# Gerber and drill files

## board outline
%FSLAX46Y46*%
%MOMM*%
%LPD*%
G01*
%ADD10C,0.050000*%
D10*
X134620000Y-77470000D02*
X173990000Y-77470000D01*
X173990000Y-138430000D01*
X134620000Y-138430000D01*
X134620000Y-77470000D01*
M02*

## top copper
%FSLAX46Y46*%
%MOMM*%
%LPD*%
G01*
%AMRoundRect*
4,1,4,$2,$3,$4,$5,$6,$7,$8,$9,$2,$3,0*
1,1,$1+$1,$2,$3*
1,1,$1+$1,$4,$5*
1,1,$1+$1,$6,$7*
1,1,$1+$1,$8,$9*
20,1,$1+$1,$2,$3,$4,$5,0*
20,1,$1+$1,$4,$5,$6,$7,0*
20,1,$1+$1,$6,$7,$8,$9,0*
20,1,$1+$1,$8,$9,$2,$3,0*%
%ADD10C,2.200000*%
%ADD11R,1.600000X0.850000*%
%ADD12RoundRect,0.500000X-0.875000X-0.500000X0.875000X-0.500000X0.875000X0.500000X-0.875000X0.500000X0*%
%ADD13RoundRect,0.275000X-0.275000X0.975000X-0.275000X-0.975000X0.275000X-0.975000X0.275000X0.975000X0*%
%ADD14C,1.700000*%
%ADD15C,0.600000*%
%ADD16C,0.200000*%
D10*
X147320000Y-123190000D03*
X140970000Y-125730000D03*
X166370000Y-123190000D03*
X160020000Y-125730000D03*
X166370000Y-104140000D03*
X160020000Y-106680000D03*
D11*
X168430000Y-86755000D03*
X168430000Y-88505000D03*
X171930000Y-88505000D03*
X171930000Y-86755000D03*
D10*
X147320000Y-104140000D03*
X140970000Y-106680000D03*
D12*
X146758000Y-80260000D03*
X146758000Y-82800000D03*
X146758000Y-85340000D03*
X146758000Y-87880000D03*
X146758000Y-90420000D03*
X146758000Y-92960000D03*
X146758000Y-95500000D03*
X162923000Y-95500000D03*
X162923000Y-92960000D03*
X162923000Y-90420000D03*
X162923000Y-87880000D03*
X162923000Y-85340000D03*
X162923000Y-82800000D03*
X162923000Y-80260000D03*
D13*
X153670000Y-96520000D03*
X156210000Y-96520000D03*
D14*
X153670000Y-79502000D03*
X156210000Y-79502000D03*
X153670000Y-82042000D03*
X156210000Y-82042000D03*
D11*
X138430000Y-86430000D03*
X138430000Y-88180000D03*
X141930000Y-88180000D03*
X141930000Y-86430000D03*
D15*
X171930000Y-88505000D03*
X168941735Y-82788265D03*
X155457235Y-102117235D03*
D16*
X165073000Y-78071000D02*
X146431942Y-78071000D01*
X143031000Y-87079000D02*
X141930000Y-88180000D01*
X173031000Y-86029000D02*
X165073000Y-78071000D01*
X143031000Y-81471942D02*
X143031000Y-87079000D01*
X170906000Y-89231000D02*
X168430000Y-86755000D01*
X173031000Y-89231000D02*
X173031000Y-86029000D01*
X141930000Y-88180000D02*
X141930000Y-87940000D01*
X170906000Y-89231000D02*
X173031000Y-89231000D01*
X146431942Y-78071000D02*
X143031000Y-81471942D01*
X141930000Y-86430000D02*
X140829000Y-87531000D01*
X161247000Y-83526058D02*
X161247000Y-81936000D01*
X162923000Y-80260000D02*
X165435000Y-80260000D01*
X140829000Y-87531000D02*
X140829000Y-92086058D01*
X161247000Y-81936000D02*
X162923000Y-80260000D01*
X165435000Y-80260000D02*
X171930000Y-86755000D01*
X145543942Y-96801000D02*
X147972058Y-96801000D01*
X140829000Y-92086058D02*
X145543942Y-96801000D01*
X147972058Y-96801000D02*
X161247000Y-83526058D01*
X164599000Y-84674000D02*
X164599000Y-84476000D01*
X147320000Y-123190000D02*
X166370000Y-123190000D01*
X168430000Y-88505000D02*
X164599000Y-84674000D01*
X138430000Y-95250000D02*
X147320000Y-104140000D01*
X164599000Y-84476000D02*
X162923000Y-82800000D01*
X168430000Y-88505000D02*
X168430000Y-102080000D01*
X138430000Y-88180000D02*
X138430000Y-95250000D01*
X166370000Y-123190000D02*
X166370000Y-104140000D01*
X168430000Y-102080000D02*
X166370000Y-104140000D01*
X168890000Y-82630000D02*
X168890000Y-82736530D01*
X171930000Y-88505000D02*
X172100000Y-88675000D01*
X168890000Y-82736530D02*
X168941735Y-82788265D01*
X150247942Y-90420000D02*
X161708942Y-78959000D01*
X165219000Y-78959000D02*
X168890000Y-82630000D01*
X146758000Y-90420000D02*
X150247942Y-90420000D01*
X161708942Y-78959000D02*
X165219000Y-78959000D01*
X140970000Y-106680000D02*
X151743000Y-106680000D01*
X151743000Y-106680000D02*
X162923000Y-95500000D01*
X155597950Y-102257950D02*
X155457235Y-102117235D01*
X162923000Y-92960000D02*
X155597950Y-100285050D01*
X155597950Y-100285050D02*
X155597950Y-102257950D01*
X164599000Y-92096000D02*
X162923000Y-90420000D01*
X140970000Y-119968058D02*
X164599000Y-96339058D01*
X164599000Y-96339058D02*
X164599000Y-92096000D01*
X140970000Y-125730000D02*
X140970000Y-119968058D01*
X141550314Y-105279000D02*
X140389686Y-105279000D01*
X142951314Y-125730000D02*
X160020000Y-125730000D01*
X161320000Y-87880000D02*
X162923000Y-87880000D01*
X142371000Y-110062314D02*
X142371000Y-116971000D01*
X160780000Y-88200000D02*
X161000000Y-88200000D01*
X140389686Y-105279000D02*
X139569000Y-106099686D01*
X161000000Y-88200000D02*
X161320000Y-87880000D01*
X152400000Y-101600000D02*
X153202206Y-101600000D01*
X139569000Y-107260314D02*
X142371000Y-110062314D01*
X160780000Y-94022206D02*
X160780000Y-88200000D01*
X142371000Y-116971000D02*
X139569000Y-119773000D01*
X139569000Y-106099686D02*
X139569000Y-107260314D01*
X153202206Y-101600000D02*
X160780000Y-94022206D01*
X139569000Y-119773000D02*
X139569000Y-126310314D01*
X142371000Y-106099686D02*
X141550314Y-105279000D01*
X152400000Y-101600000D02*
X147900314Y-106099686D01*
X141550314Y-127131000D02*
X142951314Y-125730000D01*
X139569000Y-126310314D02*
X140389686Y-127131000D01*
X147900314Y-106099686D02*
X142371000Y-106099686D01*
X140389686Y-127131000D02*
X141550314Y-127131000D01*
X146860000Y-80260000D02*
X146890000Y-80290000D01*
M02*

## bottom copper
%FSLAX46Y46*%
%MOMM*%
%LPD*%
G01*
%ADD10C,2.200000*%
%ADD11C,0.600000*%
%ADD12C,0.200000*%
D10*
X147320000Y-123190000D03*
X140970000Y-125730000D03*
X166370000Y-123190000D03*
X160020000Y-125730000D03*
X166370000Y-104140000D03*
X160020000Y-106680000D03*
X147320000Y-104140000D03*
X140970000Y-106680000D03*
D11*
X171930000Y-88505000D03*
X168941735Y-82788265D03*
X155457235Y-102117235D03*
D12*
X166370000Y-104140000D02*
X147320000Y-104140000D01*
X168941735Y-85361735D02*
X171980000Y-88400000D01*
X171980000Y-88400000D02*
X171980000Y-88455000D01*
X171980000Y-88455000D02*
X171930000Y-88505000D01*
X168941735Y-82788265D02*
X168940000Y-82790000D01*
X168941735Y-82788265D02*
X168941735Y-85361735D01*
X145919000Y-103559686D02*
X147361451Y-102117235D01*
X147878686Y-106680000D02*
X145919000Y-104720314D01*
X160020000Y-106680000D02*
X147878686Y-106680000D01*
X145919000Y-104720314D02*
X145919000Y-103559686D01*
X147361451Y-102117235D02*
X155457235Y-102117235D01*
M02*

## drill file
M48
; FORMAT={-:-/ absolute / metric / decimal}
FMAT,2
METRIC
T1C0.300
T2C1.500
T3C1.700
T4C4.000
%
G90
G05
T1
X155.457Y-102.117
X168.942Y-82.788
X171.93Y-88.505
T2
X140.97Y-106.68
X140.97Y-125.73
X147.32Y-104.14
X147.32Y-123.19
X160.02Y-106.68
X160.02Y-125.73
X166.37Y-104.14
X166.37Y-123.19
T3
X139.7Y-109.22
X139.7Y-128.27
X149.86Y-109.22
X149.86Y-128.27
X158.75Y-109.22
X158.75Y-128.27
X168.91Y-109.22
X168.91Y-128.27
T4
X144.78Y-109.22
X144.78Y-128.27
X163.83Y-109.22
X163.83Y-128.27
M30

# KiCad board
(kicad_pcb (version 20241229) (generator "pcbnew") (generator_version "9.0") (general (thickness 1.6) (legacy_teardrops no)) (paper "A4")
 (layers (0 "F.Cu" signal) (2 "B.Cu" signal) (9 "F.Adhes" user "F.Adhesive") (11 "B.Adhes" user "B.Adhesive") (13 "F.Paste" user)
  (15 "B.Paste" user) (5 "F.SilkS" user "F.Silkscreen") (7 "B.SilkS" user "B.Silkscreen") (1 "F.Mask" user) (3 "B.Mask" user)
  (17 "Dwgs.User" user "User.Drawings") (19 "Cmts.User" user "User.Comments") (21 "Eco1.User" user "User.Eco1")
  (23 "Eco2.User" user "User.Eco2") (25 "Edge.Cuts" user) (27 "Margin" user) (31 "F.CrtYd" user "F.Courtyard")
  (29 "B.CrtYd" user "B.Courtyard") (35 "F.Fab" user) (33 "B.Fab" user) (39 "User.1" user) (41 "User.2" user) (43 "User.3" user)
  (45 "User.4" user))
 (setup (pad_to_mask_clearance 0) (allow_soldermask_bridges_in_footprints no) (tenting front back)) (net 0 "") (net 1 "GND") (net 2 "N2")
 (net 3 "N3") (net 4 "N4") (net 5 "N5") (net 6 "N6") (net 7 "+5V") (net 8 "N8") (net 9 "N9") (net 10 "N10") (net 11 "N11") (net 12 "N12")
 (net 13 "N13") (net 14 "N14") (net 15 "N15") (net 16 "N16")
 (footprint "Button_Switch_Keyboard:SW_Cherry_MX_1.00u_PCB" (layer "F.Cu") (at 147.32 123.19)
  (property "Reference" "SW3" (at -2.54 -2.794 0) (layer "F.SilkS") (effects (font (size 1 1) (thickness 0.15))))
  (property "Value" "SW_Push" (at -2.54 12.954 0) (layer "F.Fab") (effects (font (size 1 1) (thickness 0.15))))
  (pad "" np_thru_hole circle (at -7.62 5.08) (size 1.7 1.7) (drill 1.7) (layers "*.Cu" "*.Mask"))
  (pad "" np_thru_hole circle (at -2.54 5.08) (size 4 4) (drill 4) (layers "*.Cu" "*.Mask"))
  (pad "" np_thru_hole circle (at 2.54 5.08) (size 1.7 1.7) (drill 1.7) (layers "*.Cu" "*.Mask"))
  (pad "1" thru_hole circle (at 0 0) (size 2.2 2.2) (drill 1.5) (layers "*.Cu" "*.Mask") (remove_unused_layers no) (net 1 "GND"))
  (pad "2" thru_hole circle (at -6.35 2.54) (size 2.2 2.2) (drill 1.5) (layers "*.Cu" "*.Mask") (remove_unused_layers no) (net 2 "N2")))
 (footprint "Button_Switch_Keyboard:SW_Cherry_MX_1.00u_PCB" (layer "F.Cu") (at 166.37 123.19)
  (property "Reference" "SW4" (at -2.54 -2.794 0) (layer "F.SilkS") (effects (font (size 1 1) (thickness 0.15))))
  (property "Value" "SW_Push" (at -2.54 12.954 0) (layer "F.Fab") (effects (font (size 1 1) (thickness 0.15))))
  (pad "" np_thru_hole circle (at -7.62 5.08) (size 1.7 1.7) (drill 1.7) (layers "*.Cu" "*.Mask"))
  (pad "" np_thru_hole circle (at -2.54 5.08) (size 4 4) (drill 4) (layers "*.Cu" "*.Mask"))
  (pad "" np_thru_hole circle (at 2.54 5.08) (size 1.7 1.7) (drill 1.7) (layers "*.Cu" "*.Mask"))
  (pad "1" thru_hole circle (at 0 0) (size 2.2 2.2) (drill 1.5) (layers "*.Cu" "*.Mask") (remove_unused_layers no) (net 1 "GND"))
  (pad "2" thru_hole circle (at -6.35 2.54) (size 2.2 2.2) (drill 1.5) (layers "*.Cu" "*.Mask") (remove_unused_layers no) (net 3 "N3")))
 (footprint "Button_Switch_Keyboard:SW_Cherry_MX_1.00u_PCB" (layer "F.Cu") (at 166.37 104.14)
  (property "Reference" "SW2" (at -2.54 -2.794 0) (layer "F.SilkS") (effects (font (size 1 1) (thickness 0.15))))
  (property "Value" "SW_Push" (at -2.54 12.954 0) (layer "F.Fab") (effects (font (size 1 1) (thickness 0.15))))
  (pad "" np_thru_hole circle (at -7.62 5.08) (size 1.7 1.7) (drill 1.7) (layers "*.Cu" "*.Mask"))
  (pad "" np_thru_hole circle (at -2.54 5.08) (size 4 4) (drill 4) (layers "*.Cu" "*.Mask"))
  (pad "" np_thru_hole circle (at 2.54 5.08) (size 1.7 1.7) (drill 1.7) (layers "*.Cu" "*.Mask"))
  (pad "1" thru_hole circle (at 0 0) (size 2.2 2.2) (drill 1.5) (layers "*.Cu" "*.Mask") (remove_unused_layers no) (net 1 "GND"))
  (pad "2" thru_hole circle (at -6.35 2.54) (size 2.2 2.2) (drill 1.5) (layers "*.Cu" "*.Mask") (remove_unused_layers no) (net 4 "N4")))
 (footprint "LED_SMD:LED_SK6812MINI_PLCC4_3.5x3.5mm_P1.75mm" (layer "F.Cu") (at 170.18 87.63)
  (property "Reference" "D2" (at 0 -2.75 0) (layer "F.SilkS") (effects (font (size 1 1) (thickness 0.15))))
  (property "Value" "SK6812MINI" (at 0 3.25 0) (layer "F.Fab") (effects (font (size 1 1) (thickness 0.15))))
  (pad "1" smd rect (at -1.75 -0.875) (size 1.6 0.85) (layers "F.Cu" "F.Mask" "F.Paste") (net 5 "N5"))
  (pad "2" smd rect (at -1.75 0.875) (size 1.6 0.85) (layers "F.Cu" "F.Mask" "F.Paste") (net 1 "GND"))
  (pad "3" smd rect (at 1.75 0.875) (size 1.6 0.85) (layers "F.Cu" "F.Mask" "F.Paste") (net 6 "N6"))
  (pad "4" smd rect (at 1.75 -0.875) (size 1.6 0.85) (layers "F.Cu" "F.Mask" "F.Paste") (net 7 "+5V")))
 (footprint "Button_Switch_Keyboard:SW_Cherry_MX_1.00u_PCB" (layer "F.Cu") (at 147.32 104.14)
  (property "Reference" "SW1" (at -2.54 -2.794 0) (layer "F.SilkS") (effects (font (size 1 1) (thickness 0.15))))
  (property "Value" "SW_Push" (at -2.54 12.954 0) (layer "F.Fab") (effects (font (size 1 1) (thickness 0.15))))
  (pad "" np_thru_hole circle (at -7.62 5.08) (size 1.7 1.7) (drill 1.7) (layers "*.Cu" "*.Mask"))
  (pad "" np_thru_hole circle (at -2.54 5.08) (size 4 4) (drill 4) (layers "*.Cu" "*.Mask"))
  (pad "" np_thru_hole circle (at 2.54 5.08) (size 1.7 1.7) (drill 1.7) (layers "*.Cu" "*.Mask"))
  (pad "1" thru_hole circle (at 0 0) (size 2.2 2.2) (drill 1.5) (layers "*.Cu" "*.Mask") (remove_unused_layers no) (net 1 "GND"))
  (pad "2" thru_hole circle (at -6.35 2.54) (size 2.2 2.2) (drill 1.5) (layers "*.Cu" "*.Mask") (remove_unused_layers no) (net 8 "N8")))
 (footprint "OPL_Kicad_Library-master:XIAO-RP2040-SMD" (layer "F.Cu") (at 154.758 87.88)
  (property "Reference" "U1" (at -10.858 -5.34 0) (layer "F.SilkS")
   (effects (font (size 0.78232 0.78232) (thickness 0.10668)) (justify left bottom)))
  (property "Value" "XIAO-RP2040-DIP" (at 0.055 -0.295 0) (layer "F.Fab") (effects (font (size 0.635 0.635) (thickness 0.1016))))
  (pad "1" smd roundrect (at -8 -7.62) (size 2.75 2) (layers "F.Cu" "F.Mask" "F.Paste") (roundrect_rratio 0.25) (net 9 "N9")
   (solder_mask_margin 0.0508) (thermal_bridge_angle 45))
  (pad "2" smd roundrect (at -8 -5.08) (size 2.75 2) (layers "F.Cu" "F.Mask" "F.Paste") (roundrect_rratio 0.25) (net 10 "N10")
   (solder_mask_margin 0.0508) (thermal_bridge_angle 45))
  (pad "3" smd roundrect (at -8 -2.54) (size 2.75 2) (layers "F.Cu" "F.Mask" "F.Paste") (roundrect_rratio 0.25) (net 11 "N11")
   (solder_mask_margin 0.0508) (thermal_bridge_angle 45))
  (pad "4" smd roundrect (at -8 0) (size 2.75 2) (layers "F.Cu" "F.Mask" "F.Paste") (roundrect_rratio 0.25) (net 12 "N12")
   (solder_mask_margin 0.0508) (thermal_bridge_angle 45))
  (pad "5" smd roundrect (at -8 2.54) (size 2.75 2) (layers "F.Cu" "F.Mask" "F.Paste") (roundrect_rratio 0.25) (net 6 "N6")
   (solder_mask_margin 0.0508) (thermal_bridge_angle 45))
  (pad "6" smd roundrect (at -8 5.08) (size 2.75 2) (layers "F.Cu" "F.Mask" "F.Paste") (roundrect_rratio 0.25) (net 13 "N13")
   (solder_mask_margin 0.0508) (thermal_bridge_angle 45))
  (pad "7" smd roundrect (at -8 7.62) (size 2.75 2) (layers "F.Cu" "F.Mask" "F.Paste") (roundrect_rratio 0.25) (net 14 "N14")
   (solder_mask_margin 0.0508) (thermal_bridge_angle 45))
  (pad "8" smd roundrect (at 8.165 7.62) (size 2.75 2) (layers "F.Cu" "F.Mask" "F.Paste") (roundrect_rratio 0.25) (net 8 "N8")
   (solder_mask_margin 0.0508) (thermal_bridge_angle 45))
  (pad "9" smd roundrect (at 8.165 5.08) (size 2.75 2) (layers "F.Cu" "F.Mask" "F.Paste") (roundrect_rratio 0.25) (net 4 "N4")
   (solder_mask_margin 0.0508) (thermal_bridge_angle 45))
  (pad "10" smd roundrect (at 8.165 2.54) (size 2.75 2) (layers "F.Cu" "F.Mask" "F.Paste") (roundrect_rratio 0.25) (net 2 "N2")
   (solder_mask_margin 0.0508) (thermal_bridge_angle 45))
  (pad "11" smd roundrect (at 8.165 0) (size 2.75 2) (layers "F.Cu" "F.Mask" "F.Paste") (roundrect_rratio 0.25) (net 3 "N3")
   (solder_mask_margin 0.0508) (thermal_bridge_angle 45))
  (pad "12" smd roundrect (at 8.165 -2.54) (size 2.75 2) (layers "F.Cu" "F.Mask" "F.Paste") (roundrect_rratio 0.25) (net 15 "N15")
   (solder_mask_margin 0.0508) (thermal_bridge_angle 45))
  (pad "13" smd roundrect (at 8.165 -5.08) (size 2.75 2) (layers "F.Cu" "F.Mask" "F.Paste") (roundrect_rratio 0.25) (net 1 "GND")
   (solder_mask_margin 0.0508) (thermal_bridge_angle 45))
  (pad "14" smd roundrect (at 8.165 -7.62) (size 2.75 2) (layers "F.Cu" "F.Mask" "F.Paste") (roundrect_rratio 0.25) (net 7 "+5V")
   (solder_mask_margin 0.0508) (thermal_bridge_angle 45))
  (pad "15" smd roundrect (at -1.088 8.64 270) (size 2.5 1.1) (layers "F.Cu" "F.Mask" "F.Paste") (roundrect_rratio 0.25)
   (thermal_bridge_angle 45))
  (pad "16" smd roundrect (at 1.452 8.64 270) (size 2.5 1.1) (layers "F.Cu" "F.Mask" "F.Paste") (roundrect_rratio 0.25)
   (thermal_bridge_angle 45))
  (pad "17" smd circle (at -1.088 -8.378) (size 1.7 1.7) (layers "F.Cu" "F.Mask" "F.Paste"))
  (pad "18" smd circle (at 1.452 -8.378) (size 1.7 1.7) (layers "F.Cu" "F.Mask" "F.Paste"))
  (pad "19" smd circle (at -1.088 -5.838) (size 1.7 1.7) (layers "F.Cu" "F.Mask" "F.Paste"))
  (pad "20" smd circle (at 1.452 -5.838) (size 1.7 1.7) (layers "F.Cu" "F.Mask" "F.Paste")))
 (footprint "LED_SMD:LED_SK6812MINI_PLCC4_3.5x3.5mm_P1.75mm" (layer "F.Cu") (at 140.18 87.305)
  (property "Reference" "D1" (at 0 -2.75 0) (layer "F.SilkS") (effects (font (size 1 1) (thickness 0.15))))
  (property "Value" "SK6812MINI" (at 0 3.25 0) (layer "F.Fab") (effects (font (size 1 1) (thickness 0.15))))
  (pad "1" smd rect (at -1.75 -0.875) (size 1.6 0.85) (layers "F.Cu" "F.Mask" "F.Paste") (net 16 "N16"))
  (pad "2" smd rect (at -1.75 0.875) (size 1.6 0.85) (layers "F.Cu" "F.Mask" "F.Paste") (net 1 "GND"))
  (pad "3" smd rect (at 1.75 0.875) (size 1.6 0.85) (layers "F.Cu" "F.Mask" "F.Paste") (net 5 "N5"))
  (pad "4" smd rect (at 1.75 -0.875) (size 1.6 0.85) (layers "F.Cu" "F.Mask" "F.Paste") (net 7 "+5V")))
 (gr_rect (start 134.62 77.47) (end 173.99 138.43) (stroke (width 0.05) (type default)) (fill no) (layer "Edge.Cuts"))
 (segment (start 165.073 78.071) (end 146.431942 78.071) (width 0.2) (layer "F.Cu") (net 5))
 (segment (start 143.031 87.079) (end 141.93 88.18) (width 0.2) (layer "F.Cu") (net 5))
 (segment (start 173.031 86.029) (end 165.073 78.071) (width 0.2) (layer "F.Cu") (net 5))
 (segment (start 143.031 81.471942) (end 143.031 87.079) (width 0.2) (layer "F.Cu") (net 5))
 (segment (start 170.906 89.231) (end 168.43 86.755) (width 0.2) (layer "F.Cu") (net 5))
 (segment (start 173.031 89.231) (end 173.031 86.029) (width 0.2) (layer "F.Cu") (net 5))
 (segment (start 141.93 88.18) (end 141.93 87.94) (width 0.2) (layer "F.Cu") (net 5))
 (segment (start 170.906 89.231) (end 173.031 89.231) (width 0.2) (layer "F.Cu") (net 5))
 (segment (start 146.431942 78.071) (end 143.031 81.471942) (width 0.2) (layer "F.Cu") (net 5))
 (segment (start 141.93 86.43) (end 140.829 87.531) (width 0.2) (layer "F.Cu") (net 7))
 (segment (start 161.247 83.526058) (end 161.247 81.936) (width 0.2) (layer "F.Cu") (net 7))
 (segment (start 162.923 80.26) (end 165.435 80.26) (width 0.2) (layer "F.Cu") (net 7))
 (segment (start 140.829 87.531) (end 140.829 92.086058) (width 0.2) (layer "F.Cu") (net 7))
 (segment (start 161.247 81.936) (end 162.923 80.26) (width 0.2) (layer "F.Cu") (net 7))
 (segment (start 165.435 80.26) (end 171.93 86.755) (width 0.2) (layer "F.Cu") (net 7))
 (segment (start 145.543942 96.801) (end 147.972058 96.801) (width 0.2) (layer "F.Cu") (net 7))
 (segment (start 140.829 92.086058) (end 145.543942 96.801) (width 0.2) (layer "F.Cu") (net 7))
 (segment (start 147.972058 96.801) (end 161.247 83.526058) (width 0.2) (layer "F.Cu") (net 7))
 (segment (start 164.599 84.674) (end 164.599 84.476) (width 0.2) (layer "F.Cu") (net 1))
 (segment (start 147.32 123.19) (end 166.37 123.19) (width 0.2) (layer "F.Cu") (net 1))
 (segment (start 168.43 88.505) (end 164.599 84.674) (width 0.2) (layer "F.Cu") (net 1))
 (segment (start 138.43 95.25) (end 147.32 104.14) (width 0.2) (layer "F.Cu") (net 1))
 (segment (start 164.599 84.476) (end 162.923 82.8) (width 0.2) (layer "F.Cu") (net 1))
 (segment (start 168.43 88.505) (end 168.43 102.08) (width 0.2) (layer "F.Cu") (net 1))
 (segment (start 138.43 88.18) (end 138.43 95.25) (width 0.2) (layer "F.Cu") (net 1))
 (segment (start 166.37 123.19) (end 166.37 104.14) (width 0.2) (layer "F.Cu") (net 1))
 (segment (start 168.43 102.08) (end 166.37 104.14) (width 0.2) (layer "F.Cu") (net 1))
 (segment (start 166.37 104.14) (end 147.32 104.14) (width 0.2) (layer "B.Cu") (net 1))
 (segment (start 168.89 82.63) (end 168.89 82.73653) (width 0.2) (layer "F.Cu") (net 6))
 (segment (start 171.93 88.505) (end 172.1 88.675) (width 0.2) (layer "F.Cu") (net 6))
 (segment (start 168.89 82.73653) (end 168.941735 82.788265) (width 0.2) (layer "F.Cu") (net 6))
 (segment (start 150.247942 90.42) (end 161.708942 78.959) (width 0.2) (layer "F.Cu") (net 6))
 (segment (start 165.219 78.959) (end 168.89 82.63) (width 0.2) (layer "F.Cu") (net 6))
 (segment (start 146.758 90.42) (end 150.247942 90.42) (width 0.2) (layer "F.Cu") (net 6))
 (segment (start 161.708942 78.959) (end 165.219 78.959) (width 0.2) (layer "F.Cu") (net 6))
 (via (at 171.93 88.505) (size 0.6) (drill 0.3) (layers "F.Cu" "B.Cu") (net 6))
 (via (at 168.941735 82.788265) (size 0.6) (drill 0.3) (layers "F.Cu" "B.Cu") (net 6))
 (segment (start 168.941735 85.361735) (end 171.98 88.4) (width 0.2) (layer "B.Cu") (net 6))
 (segment (start 171.98 88.4) (end 171.98 88.455) (width 0.2) (layer "B.Cu") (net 6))
 (segment (start 171.98 88.455) (end 171.93 88.505) (width 0.2) (layer "B.Cu") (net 6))
 (segment (start 168.941735 82.788265) (end 168.94 82.79) (width 0.2) (layer "B.Cu") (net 6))
 (segment (start 168.941735 82.788265) (end 168.941735 85.361735) (width 0.2) (layer "B.Cu") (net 6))
 (segment (start 140.97 106.68) (end 151.743 106.68) (width 0.2) (layer "F.Cu") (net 8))
 (segment (start 151.743 106.68) (end 162.923 95.5) (width 0.2) (layer "F.Cu") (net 8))
 (segment (start 155.59795 102.25795) (end 155.457235 102.117235) (width 0.2) (layer "F.Cu") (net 4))
 (segment (start 162.923 92.96) (end 155.59795 100.28505) (width 0.2) (layer "F.Cu") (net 4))
 (segment (start 155.59795 100.28505) (end 155.59795 102.25795) (width 0.2) (layer "F.Cu") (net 4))
 (via (at 155.457235 102.117235) (size 0.6) (drill 0.3) (layers "F.Cu" "B.Cu") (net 4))
 (segment (start 145.919 103.559686) (end 147.361451 102.117235) (width 0.2) (layer "B.Cu") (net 4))
 (segment (start 147.878686 106.68) (end 145.919 104.720314) (width 0.2) (layer "B.Cu") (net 4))
 (segment (start 160.02 106.68) (end 147.878686 106.68) (width 0.2) (layer "B.Cu") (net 4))
 (segment (start 145.919 104.720314) (end 145.919 103.559686) (width 0.2) (layer "B.Cu") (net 4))
 (segment (start 147.361451 102.117235) (end 155.457235 102.117235) (width 0.2) (layer "B.Cu") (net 4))
 (segment (start 164.599 92.096) (end 162.923 90.42) (width 0.2) (layer "F.Cu") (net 2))
 (segment (start 140.97 119.968058) (end 164.599 96.339058) (width 0.2) (layer "F.Cu") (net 2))
 (segment (start 164.599 96.339058) (end 164.599 92.096) (width 0.2) (layer "F.Cu") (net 2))
 (segment (start 140.97 125.73) (end 140.97 119.968058) (width 0.2) (layer "F.Cu") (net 2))
 (segment (start 141.550314 105.279) (end 140.389686 105.279) (width 0.2) (layer "F.Cu") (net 3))
 (segment (start 142.951314 125.73) (end 160.02 125.73) (width 0.2) (layer "F.Cu") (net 3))
 (segment (start 161.32 87.88) (end 162.923 87.88) (width 0.2) (layer "F.Cu") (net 3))
 (segment (start 142.371 110.062314) (end 142.371 116.971) (width 0.2) (layer "F.Cu") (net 3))
 (segment (start 160.78 88.2) (end 161 88.2) (width 0.2) (layer "F.Cu") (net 3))
 (segment (start 140.389686 105.279) (end 139.569 106.099686) (width 0.2) (layer "F.Cu") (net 3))
 (segment (start 161 88.2) (end 161.32 87.88) (width 0.2) (layer "F.Cu") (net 3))
 (segment (start 152.4 101.6) (end 153.202206 101.6) (width 0.2) (layer "F.Cu") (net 3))
 (segment (start 139.569 107.260314) (end 142.371 110.062314) (width 0.2) (layer "F.Cu") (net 3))
 (segment (start 160.78 94.022206) (end 160.78 88.2) (width 0.2) (layer "F.Cu") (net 3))
 (segment (start 142.371 116.971) (end 139.569 119.773) (width 0.2) (layer "F.Cu") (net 3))
 (segment (start 139.569 106.099686) (end 139.569 107.260314) (width 0.2) (layer "F.Cu") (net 3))
 (segment (start 153.202206 101.6) (end 160.78 94.022206) (width 0.2) (layer "F.Cu") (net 3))
 (segment (start 139.569 119.773) (end 139.569 126.310314) (width 0.2) (layer "F.Cu") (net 3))
 (segment (start 142.371 106.099686) (end 141.550314 105.279) (width 0.2) (layer "F.Cu") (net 3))
 (segment (start 152.4 101.6) (end 147.900314 106.099686) (width 0.2) (layer "F.Cu") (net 3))
 (segment (start 141.550314 127.131) (end 142.951314 125.73) (width 0.2) (layer "F.Cu") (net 3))
 (segment (start 139.569 126.310314) (end 140.389686 127.131) (width 0.2) (layer "F.Cu") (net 3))
 (segment (start 147.900314 106.099686) (end 142.371 106.099686) (width 0.2) (layer "F.Cu") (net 3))
 (segment (start 140.389686 127.131) (end 141.550314 127.131) (width 0.2) (layer "F.Cu") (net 3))
 (segment (start 146.86 80.26) (end 146.89 80.29) (width 0.2) (layer "F.Cu") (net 9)))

